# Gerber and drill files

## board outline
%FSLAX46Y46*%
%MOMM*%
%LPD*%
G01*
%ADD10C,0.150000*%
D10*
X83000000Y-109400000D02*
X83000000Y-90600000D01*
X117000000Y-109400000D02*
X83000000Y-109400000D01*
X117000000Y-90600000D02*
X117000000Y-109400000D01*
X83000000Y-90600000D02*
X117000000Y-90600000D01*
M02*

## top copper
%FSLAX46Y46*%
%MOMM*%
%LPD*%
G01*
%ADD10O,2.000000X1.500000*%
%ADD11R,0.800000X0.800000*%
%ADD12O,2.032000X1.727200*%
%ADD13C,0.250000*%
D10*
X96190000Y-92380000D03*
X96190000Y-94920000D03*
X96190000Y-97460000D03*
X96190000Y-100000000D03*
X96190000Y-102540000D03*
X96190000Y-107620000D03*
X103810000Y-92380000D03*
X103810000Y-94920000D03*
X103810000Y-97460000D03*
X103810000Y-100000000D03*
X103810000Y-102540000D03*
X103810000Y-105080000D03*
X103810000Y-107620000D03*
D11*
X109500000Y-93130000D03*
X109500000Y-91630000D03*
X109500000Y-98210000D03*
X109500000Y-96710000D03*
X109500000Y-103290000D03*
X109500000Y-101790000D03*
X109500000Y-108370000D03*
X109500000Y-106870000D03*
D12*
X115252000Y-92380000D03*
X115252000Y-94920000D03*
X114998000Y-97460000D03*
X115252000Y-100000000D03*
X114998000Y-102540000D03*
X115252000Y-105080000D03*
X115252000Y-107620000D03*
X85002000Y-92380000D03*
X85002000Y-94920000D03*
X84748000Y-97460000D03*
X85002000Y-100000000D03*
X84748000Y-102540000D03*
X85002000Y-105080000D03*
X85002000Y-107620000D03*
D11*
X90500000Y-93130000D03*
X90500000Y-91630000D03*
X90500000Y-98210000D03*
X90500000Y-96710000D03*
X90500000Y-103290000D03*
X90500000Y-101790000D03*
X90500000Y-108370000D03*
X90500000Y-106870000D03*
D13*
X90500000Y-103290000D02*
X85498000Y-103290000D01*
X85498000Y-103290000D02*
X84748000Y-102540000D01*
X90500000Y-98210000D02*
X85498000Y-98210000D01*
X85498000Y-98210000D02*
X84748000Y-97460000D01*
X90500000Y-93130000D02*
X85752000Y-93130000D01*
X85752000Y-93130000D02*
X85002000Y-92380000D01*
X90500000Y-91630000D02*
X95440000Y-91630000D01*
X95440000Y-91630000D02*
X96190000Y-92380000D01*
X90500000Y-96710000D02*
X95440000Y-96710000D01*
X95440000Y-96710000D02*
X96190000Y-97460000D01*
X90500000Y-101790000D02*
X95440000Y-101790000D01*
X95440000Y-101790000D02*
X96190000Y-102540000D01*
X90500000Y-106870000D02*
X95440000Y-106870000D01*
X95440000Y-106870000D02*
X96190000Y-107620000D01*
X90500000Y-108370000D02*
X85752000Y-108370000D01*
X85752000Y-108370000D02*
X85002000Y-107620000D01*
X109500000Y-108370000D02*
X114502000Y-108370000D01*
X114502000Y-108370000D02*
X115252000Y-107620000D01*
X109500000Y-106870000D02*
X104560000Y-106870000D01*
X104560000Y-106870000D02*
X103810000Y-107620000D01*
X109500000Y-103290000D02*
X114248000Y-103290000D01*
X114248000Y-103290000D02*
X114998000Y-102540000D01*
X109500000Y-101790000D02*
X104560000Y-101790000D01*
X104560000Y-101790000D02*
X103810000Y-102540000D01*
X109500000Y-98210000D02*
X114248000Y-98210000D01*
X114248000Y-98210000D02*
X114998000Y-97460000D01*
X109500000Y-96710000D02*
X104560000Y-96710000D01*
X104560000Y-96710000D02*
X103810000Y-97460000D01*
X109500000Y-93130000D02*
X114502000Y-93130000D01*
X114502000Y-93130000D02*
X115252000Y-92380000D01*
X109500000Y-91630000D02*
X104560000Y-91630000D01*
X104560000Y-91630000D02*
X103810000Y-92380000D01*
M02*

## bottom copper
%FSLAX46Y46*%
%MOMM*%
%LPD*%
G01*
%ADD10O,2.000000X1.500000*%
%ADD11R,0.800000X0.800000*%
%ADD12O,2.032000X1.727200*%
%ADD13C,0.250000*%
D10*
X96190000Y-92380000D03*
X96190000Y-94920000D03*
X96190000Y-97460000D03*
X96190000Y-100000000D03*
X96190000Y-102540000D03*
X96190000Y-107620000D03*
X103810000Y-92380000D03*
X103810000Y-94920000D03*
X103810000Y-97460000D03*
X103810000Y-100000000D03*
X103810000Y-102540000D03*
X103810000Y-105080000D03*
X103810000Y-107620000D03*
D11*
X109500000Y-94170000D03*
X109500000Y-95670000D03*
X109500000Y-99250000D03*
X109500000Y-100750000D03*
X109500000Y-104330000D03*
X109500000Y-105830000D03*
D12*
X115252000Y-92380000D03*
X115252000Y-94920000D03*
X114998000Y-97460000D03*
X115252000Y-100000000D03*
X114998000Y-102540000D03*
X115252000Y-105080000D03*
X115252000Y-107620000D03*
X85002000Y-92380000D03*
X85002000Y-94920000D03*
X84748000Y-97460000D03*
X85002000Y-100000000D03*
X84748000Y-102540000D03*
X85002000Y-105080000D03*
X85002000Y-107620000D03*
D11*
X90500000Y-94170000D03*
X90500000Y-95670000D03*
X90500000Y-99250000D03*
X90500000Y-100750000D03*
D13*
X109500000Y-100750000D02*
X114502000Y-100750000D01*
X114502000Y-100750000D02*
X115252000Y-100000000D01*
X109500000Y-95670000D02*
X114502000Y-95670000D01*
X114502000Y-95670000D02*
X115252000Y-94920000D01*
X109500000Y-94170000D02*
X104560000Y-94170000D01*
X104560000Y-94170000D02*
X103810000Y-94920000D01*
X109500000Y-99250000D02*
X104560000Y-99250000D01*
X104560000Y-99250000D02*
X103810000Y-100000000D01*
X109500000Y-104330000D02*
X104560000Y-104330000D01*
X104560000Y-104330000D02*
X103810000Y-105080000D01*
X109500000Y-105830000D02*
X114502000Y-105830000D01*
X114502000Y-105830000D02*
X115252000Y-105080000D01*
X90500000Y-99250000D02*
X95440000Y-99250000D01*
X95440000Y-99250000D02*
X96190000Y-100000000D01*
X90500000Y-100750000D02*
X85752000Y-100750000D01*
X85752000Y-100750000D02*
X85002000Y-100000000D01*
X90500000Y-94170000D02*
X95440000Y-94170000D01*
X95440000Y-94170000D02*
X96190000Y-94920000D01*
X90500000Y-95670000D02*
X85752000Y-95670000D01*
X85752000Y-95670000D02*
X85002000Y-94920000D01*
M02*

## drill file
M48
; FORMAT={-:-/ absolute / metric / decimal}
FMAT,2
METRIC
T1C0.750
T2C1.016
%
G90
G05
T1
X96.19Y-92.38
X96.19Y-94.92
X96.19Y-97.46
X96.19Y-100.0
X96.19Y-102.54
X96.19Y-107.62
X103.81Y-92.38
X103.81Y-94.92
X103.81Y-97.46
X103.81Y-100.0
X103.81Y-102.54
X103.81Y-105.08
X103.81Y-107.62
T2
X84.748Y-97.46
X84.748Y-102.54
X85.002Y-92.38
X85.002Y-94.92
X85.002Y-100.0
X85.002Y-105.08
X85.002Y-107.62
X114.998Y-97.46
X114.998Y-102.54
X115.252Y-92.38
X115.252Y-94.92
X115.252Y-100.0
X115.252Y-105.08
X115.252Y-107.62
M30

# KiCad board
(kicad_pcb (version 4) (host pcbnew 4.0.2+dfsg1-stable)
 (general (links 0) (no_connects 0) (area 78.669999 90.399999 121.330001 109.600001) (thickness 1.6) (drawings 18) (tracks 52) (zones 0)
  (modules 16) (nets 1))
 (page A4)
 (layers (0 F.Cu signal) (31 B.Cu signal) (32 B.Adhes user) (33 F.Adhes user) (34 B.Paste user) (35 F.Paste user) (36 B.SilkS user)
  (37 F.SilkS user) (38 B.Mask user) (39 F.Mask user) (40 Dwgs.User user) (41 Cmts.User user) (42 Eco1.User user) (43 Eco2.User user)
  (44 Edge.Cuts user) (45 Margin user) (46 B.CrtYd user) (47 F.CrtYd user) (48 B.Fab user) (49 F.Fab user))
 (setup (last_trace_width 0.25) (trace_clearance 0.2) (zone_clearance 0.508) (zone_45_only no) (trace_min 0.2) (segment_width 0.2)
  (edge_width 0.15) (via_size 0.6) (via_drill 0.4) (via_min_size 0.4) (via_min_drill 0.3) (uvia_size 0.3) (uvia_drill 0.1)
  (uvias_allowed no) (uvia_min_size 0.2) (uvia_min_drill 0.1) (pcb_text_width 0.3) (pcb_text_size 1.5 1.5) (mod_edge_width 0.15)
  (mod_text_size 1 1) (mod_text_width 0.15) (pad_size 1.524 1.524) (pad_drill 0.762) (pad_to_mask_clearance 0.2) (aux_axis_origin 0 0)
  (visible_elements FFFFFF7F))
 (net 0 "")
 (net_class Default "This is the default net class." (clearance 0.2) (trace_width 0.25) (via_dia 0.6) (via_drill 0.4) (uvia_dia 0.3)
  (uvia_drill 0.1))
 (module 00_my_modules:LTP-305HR (layer F.Cu) (at 100 100)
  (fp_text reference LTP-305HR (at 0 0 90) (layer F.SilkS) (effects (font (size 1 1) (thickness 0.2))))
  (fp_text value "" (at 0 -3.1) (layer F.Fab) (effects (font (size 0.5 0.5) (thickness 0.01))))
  (pad A2 thru_hole oval (at -3.81 -7.62) (size 2 1.5) (drill 0.75) (layers *.Cu *.Mask F.SilkS))
  (pad C1 thru_hole oval (at -3.81 -5.08) (size 2 1.5) (drill 0.75) (layers *.Cu *.Mask F.SilkS))
  (pad C3 thru_hole oval (at -3.81 -2.54) (size 2 1.5) (drill 0.75) (layers *.Cu *.Mask F.SilkS))
  (pad C4 thru_hole oval (at -3.81 0) (size 2 1.5) (drill 0.75) (layers *.Cu *.Mask F.SilkS))
  (pad A1 thru_hole oval (at -3.81 2.54) (size 2 1.5) (drill 0.75) (layers *.Cu *.Mask F.SilkS))
  (pad AD thru_hole oval (at -3.81 7.62) (size 2 1.5) (drill 0.75) (layers *.Cu *.Mask F.SilkS))
  (pad A4 thru_hole oval (at 3.81 -7.62) (size 2 1.5) (drill 0.75) (layers *.Cu *.Mask F.SilkS))
  (pad A5 thru_hole oval (at 3.81 -5.08) (size 2 1.5) (drill 0.75) (layers *.Cu *.Mask F.SilkS))
  (pad C2 thru_hole oval (at 3.81 -2.54) (size 2 1.5) (drill 0.75) (layers *.Cu *.Mask F.SilkS))
  (pad C5 thru_hole oval (at 3.81 0) (size 2 1.5) (drill 0.75) (layers *.Cu *.Mask F.SilkS))
  (pad C6 thru_hole oval (at 3.81 2.54) (size 2 1.5) (drill 0.75) (layers *.Cu *.Mask F.SilkS))
  (pad C7 thru_hole oval (at 3.81 5.08) (size 2 1.5) (drill 0.75) (layers *.Cu *.Mask F.SilkS))
  (pad A3 thru_hole oval (at 3.81 7.62) (size 2 1.5) (drill 0.75) (layers *.Cu *.Mask F.SilkS)))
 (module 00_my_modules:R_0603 (layer F.Cu) (at 109.5 92.38 90)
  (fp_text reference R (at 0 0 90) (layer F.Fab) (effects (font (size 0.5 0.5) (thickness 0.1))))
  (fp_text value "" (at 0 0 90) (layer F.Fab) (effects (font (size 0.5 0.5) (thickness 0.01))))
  (pad 1 smd rect (at -0.75 0 90) (size 0.8 0.8) (layers F.Cu F.Paste F.Mask))
  (pad 2 smd rect (at 0.75 0 90) (size 0.8 0.8) (layers F.Cu F.Paste F.Mask)))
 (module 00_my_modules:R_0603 (layer F.Cu) (at 109.5 97.46 90)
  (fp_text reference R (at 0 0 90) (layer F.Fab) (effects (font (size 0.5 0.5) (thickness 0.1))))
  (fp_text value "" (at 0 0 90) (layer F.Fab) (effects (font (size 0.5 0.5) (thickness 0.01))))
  (pad 1 smd rect (at -0.75 0 90) (size 0.8 0.8) (layers F.Cu F.Paste F.Mask))
  (pad 2 smd rect (at 0.75 0 90) (size 0.8 0.8) (layers F.Cu F.Paste F.Mask)))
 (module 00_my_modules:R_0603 (layer F.Cu) (at 109.5 102.54 90)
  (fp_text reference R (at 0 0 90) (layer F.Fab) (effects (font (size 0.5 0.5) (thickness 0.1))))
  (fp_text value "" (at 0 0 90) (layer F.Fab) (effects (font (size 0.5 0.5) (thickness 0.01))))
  (pad 1 smd rect (at -0.75 0 90) (size 0.8 0.8) (layers F.Cu F.Paste F.Mask))
  (pad 2 smd rect (at 0.75 0 90) (size 0.8 0.8) (layers F.Cu F.Paste F.Mask)))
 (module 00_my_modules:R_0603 (layer F.Cu) (at 109.5 107.62 90)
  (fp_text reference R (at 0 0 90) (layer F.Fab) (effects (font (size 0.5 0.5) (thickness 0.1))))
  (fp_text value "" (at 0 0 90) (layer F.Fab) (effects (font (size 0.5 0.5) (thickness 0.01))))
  (pad 1 smd rect (at -0.75 0 90) (size 0.8 0.8) (layers F.Cu F.Paste F.Mask))
  (pad 2 smd rect (at 0.75 0 90) (size 0.8 0.8) (layers F.Cu F.Paste F.Mask)))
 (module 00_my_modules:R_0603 (layer B.Cu) (at 109.5 94.92 270)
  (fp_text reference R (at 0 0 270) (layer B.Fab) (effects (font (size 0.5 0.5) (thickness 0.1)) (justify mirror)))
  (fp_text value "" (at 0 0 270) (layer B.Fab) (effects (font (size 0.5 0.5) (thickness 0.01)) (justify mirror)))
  (pad 1 smd rect (at -0.75 0 270) (size 0.8 0.8) (layers B.Cu B.Paste B.Mask))
  (pad 2 smd rect (at 0.75 0 270) (size 0.8 0.8) (layers B.Cu B.Paste B.Mask)))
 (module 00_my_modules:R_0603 (layer B.Cu) (at 109.5 100 270)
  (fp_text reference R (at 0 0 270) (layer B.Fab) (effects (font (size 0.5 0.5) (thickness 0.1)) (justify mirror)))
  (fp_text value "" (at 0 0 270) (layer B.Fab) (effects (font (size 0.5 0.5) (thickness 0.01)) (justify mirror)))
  (pad 1 smd rect (at -0.75 0 270) (size 0.8 0.8) (layers B.Cu B.Paste B.Mask))
  (pad 2 smd rect (at 0.75 0 270) (size 0.8 0.8) (layers B.Cu B.Paste B.Mask)))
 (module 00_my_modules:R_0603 (layer B.Cu) (at 109.5 105.08 270)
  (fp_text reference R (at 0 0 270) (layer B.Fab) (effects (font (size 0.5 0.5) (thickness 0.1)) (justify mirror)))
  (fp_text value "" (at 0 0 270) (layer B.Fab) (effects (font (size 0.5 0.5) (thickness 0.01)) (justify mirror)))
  (pad 1 smd rect (at -0.75 0 270) (size 0.8 0.8) (layers B.Cu B.Paste B.Mask))
  (pad 2 smd rect (at 0.75 0 270) (size 0.8 0.8) (layers B.Cu B.Paste B.Mask)))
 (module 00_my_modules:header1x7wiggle (layer F.Cu) (at 115.125 100)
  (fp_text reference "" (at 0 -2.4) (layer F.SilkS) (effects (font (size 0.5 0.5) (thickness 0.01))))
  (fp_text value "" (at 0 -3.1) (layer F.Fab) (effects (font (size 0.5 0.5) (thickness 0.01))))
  (pad 1 thru_hole oval (at 0.127 -7.62) (size 2.032 1.7272) (drill 1.016) (layers *.Cu *.Mask F.SilkS))
  (pad 2 thru_hole oval (at 0.127 -5.08) (size 2.032 1.7272) (drill 1.016) (layers *.Cu *.Mask F.SilkS))
  (pad 3 thru_hole oval (at -0.127 -2.54) (size 2.032 1.7272) (drill 1.016) (layers *.Cu *.Mask F.SilkS))
  (pad 4 thru_hole oval (at 0.127 0) (size 2.032 1.7272) (drill 1.016) (layers *.Cu *.Mask F.SilkS))
  (pad 5 thru_hole oval (at -0.127 2.54) (size 2.032 1.7272) (drill 1.016) (layers *.Cu *.Mask F.SilkS))
  (pad 6 thru_hole oval (at 0.127 5.08) (size 2.032 1.7272) (drill 1.016) (layers *.Cu *.Mask F.SilkS))
  (pad 7 thru_hole oval (at 0.127 7.62) (size 2.032 1.7272) (drill 1.016) (layers *.Cu *.Mask F.SilkS)))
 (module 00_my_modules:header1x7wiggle (layer F.Cu) (at 84.875 100)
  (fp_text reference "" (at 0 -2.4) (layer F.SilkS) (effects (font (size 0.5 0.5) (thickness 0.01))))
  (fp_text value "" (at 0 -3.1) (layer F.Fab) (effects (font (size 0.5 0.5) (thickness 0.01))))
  (pad 1 thru_hole oval (at 0.127 -7.62) (size 2.032 1.7272) (drill 1.016) (layers *.Cu *.Mask F.SilkS))
  (pad 2 thru_hole oval (at 0.127 -5.08) (size 2.032 1.7272) (drill 1.016) (layers *.Cu *.Mask F.SilkS))
  (pad 3 thru_hole oval (at -0.127 -2.54) (size 2.032 1.7272) (drill 1.016) (layers *.Cu *.Mask F.SilkS))
  (pad 4 thru_hole oval (at 0.127 0) (size 2.032 1.7272) (drill 1.016) (layers *.Cu *.Mask F.SilkS))
  (pad 5 thru_hole oval (at -0.127 2.54) (size 2.032 1.7272) (drill 1.016) (layers *.Cu *.Mask F.SilkS))
  (pad 6 thru_hole oval (at 0.127 5.08) (size 2.032 1.7272) (drill 1.016) (layers *.Cu *.Mask F.SilkS))
  (pad 7 thru_hole oval (at 0.127 7.62) (size 2.032 1.7272) (drill 1.016) (layers *.Cu *.Mask F.SilkS)))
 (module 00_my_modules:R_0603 (layer F.Cu) (at 90.5 92.38 90)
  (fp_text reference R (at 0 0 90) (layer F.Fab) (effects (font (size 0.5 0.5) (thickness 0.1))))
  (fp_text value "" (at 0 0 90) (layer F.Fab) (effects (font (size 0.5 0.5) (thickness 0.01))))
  (pad 1 smd rect (at -0.75 0 90) (size 0.8 0.8) (layers F.Cu F.Paste F.Mask))
  (pad 2 smd rect (at 0.75 0 90) (size 0.8 0.8) (layers F.Cu F.Paste F.Mask)))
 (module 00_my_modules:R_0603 (layer F.Cu) (at 90.5 97.46 90)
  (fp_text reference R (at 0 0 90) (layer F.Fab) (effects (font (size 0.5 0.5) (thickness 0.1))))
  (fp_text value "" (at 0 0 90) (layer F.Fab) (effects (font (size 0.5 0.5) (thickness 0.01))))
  (pad 1 smd rect (at -0.75 0 90) (size 0.8 0.8) (layers F.Cu F.Paste F.Mask))
  (pad 2 smd rect (at 0.75 0 90) (size 0.8 0.8) (layers F.Cu F.Paste F.Mask)))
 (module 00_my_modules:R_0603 (layer F.Cu) (at 90.5 102.54 90)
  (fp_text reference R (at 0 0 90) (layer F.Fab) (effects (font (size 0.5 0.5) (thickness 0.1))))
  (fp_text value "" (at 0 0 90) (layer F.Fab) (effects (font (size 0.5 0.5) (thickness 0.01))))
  (pad 1 smd rect (at -0.75 0 90) (size 0.8 0.8) (layers F.Cu F.Paste F.Mask))
  (pad 2 smd rect (at 0.75 0 90) (size 0.8 0.8) (layers F.Cu F.Paste F.Mask)))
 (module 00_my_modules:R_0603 (layer F.Cu) (at 90.5 107.62 90)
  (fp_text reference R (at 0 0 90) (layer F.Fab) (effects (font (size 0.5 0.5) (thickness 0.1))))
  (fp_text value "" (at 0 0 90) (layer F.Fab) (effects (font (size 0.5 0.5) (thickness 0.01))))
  (pad 1 smd rect (at -0.75 0 90) (size 0.8 0.8) (layers F.Cu F.Paste F.Mask))
  (pad 2 smd rect (at 0.75 0 90) (size 0.8 0.8) (layers F.Cu F.Paste F.Mask)))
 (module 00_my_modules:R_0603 (layer B.Cu) (at 90.5 94.92 270)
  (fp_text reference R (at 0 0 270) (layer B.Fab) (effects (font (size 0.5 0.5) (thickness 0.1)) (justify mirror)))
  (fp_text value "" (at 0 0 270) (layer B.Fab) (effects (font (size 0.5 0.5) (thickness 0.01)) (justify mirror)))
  (pad 1 smd rect (at -0.75 0 270) (size 0.8 0.8) (layers B.Cu B.Paste B.Mask))
  (pad 2 smd rect (at 0.75 0 270) (size 0.8 0.8) (layers B.Cu B.Paste B.Mask)))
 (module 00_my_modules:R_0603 (layer B.Cu) (at 90.5 100 270)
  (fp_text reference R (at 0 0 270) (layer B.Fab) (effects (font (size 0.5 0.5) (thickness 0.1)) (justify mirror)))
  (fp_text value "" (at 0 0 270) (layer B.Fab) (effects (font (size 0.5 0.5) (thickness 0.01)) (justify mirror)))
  (pad 1 smd rect (at -0.75 0 270) (size 0.8 0.8) (layers B.Cu B.Paste B.Mask))
  (pad 2 smd rect (at 0.75 0 270) (size 0.8 0.8) (layers B.Cu B.Paste B.Mask)))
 (gr_line (start 83 109.4) (end 83 90.6) (angle 90) (layer Edge.Cuts) (width 0.15))
 (gr_line (start 117 109.4) (end 83 109.4) (angle 90) (layer Edge.Cuts) (width 0.15))
 (gr_line (start 117 90.6) (end 117 109.4) (angle 90) (layer Edge.Cuts) (width 0.15))
 (gr_line (start 83 90.6) (end 117 90.6) (angle 90) (layer Edge.Cuts) (width 0.15))
 (segment (start 109.5 100.75) (end 114.502 100.75) (width 0.25) (layer B.Cu) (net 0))
 (segment (start 114.502 100.75) (end 115.252 100) (width 0.25) (layer B.Cu) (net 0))
 (segment (start 109.5 95.67) (end 114.502 95.67) (width 0.25) (layer B.Cu) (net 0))
 (segment (start 114.502 95.67) (end 115.252 94.92) (width 0.25) (layer B.Cu) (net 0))
 (segment (start 109.5 94.17) (end 104.56 94.17) (width 0.25) (layer B.Cu) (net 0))
 (segment (start 104.56 94.17) (end 103.81 94.92) (width 0.25) (layer B.Cu) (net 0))
 (segment (start 109.5 99.25) (end 104.56 99.25) (width 0.25) (layer B.Cu) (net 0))
 (segment (start 104.56 99.25) (end 103.81 100) (width 0.25) (layer B.Cu) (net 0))
 (segment (start 109.5 104.33) (end 104.56 104.33) (width 0.25) (layer B.Cu) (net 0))
 (segment (start 104.56 104.33) (end 103.81 105.08) (width 0.25) (layer B.Cu) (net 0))
 (segment (start 109.5 105.83) (end 114.502 105.83) (width 0.25) (layer B.Cu) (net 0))
 (segment (start 114.502 105.83) (end 115.252 105.08) (width 0.25) (layer B.Cu) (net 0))
 (segment (start 90.5 99.25) (end 95.44 99.25) (width 0.25) (layer B.Cu) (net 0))
 (segment (start 95.44 99.25) (end 96.19 100) (width 0.25) (layer B.Cu) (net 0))
 (segment (start 90.5 100.75) (end 85.752 100.75) (width 0.25) (layer B.Cu) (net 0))
 (segment (start 85.752 100.75) (end 85.002 100) (width 0.25) (layer B.Cu) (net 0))
 (segment (start 90.5 94.17) (end 95.44 94.17) (width 0.25) (layer B.Cu) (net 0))
 (segment (start 95.44 94.17) (end 96.19 94.92) (width 0.25) (layer B.Cu) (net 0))
 (segment (start 90.5 95.67) (end 85.752 95.67) (width 0.25) (layer B.Cu) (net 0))
 (segment (start 85.752 95.67) (end 85.002 94.92) (width 0.25) (layer B.Cu) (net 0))
 (segment (start 90.5 103.29) (end 85.498 103.29) (width 0.25) (layer F.Cu) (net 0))
 (segment (start 85.498 103.29) (end 84.748 102.54) (width 0.25) (layer F.Cu) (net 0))
 (segment (start 90.5 98.21) (end 85.498 98.21) (width 0.25) (layer F.Cu) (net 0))
 (segment (start 85.498 98.21) (end 84.748 97.46) (width 0.25) (layer F.Cu) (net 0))
 (segment (start 90.5 93.13) (end 85.752 93.13) (width 0.25) (layer F.Cu) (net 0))
 (segment (start 85.752 93.13) (end 85.002 92.38) (width 0.25) (layer F.Cu) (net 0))
 (segment (start 90.5 91.63) (end 95.44 91.63) (width 0.25) (layer F.Cu) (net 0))
 (segment (start 95.44 91.63) (end 96.19 92.38) (width 0.25) (layer F.Cu) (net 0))
 (segment (start 90.5 96.71) (end 95.44 96.71) (width 0.25) (layer F.Cu) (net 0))
 (segment (start 95.44 96.71) (end 96.19 97.46) (width 0.25) (layer F.Cu) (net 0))
 (segment (start 90.5 101.79) (end 95.44 101.79) (width 0.25) (layer F.Cu) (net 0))
 (segment (start 95.44 101.79) (end 96.19 102.54) (width 0.25) (layer F.Cu) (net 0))
 (segment (start 90.5 106.87) (end 95.44 106.87) (width 0.25) (layer F.Cu) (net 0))
 (segment (start 95.44 106.87) (end 96.19 107.62) (width 0.25) (layer F.Cu) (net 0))
 (segment (start 90.5 108.37) (end 85.752 108.37) (width 0.25) (layer F.Cu) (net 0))
 (segment (start 85.752 108.37) (end 85.002 107.62) (width 0.25) (layer F.Cu) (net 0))
 (segment (start 109.5 108.37) (end 114.502 108.37) (width 0.25) (layer F.Cu) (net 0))
 (segment (start 114.502 108.37) (end 115.252 107.62) (width 0.25) (layer F.Cu) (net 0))
 (segment (start 109.5 106.87) (end 104.56 106.87) (width 0.25) (layer F.Cu) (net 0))
 (segment (start 104.56 106.87) (end 103.81 107.62) (width 0.25) (layer F.Cu) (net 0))
 (segment (start 109.5 103.29) (end 114.248 103.29) (width 0.25) (layer F.Cu) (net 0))
 (segment (start 114.248 103.29) (end 114.998 102.54) (width 0.25) (layer F.Cu) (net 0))
 (segment (start 109.5 101.79) (end 104.56 101.79) (width 0.25) (layer F.Cu) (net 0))
 (segment (start 104.56 101.79) (end 103.81 102.54) (width 0.25) (layer F.Cu) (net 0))
 (segment (start 109.5 98.21) (end 114.248 98.21) (width 0.25) (layer F.Cu) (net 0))
 (segment (start 114.248 98.21) (end 114.998 97.46) (width 0.25) (layer F.Cu) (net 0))
 (segment (start 109.5 96.71) (end 104.56 96.71) (width 0.25) (layer F.Cu) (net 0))
 (segment (start 104.56 96.71) (end 103.81 97.46) (width 0.25) (layer F.Cu) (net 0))
 (segment (start 109.5 93.13) (end 114.502 93.13) (width 0.25) (layer F.Cu) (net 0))
 (segment (start 114.502 93.13) (end 115.252 92.38) (width 0.25) (layer F.Cu) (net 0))
 (segment (start 109.5 91.63) (end 104.56 91.63) (width 0.25) (layer F.Cu) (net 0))
 (segment (start 104.56 91.63) (end 103.81 92.38) (width 0.25) (layer F.Cu) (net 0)))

